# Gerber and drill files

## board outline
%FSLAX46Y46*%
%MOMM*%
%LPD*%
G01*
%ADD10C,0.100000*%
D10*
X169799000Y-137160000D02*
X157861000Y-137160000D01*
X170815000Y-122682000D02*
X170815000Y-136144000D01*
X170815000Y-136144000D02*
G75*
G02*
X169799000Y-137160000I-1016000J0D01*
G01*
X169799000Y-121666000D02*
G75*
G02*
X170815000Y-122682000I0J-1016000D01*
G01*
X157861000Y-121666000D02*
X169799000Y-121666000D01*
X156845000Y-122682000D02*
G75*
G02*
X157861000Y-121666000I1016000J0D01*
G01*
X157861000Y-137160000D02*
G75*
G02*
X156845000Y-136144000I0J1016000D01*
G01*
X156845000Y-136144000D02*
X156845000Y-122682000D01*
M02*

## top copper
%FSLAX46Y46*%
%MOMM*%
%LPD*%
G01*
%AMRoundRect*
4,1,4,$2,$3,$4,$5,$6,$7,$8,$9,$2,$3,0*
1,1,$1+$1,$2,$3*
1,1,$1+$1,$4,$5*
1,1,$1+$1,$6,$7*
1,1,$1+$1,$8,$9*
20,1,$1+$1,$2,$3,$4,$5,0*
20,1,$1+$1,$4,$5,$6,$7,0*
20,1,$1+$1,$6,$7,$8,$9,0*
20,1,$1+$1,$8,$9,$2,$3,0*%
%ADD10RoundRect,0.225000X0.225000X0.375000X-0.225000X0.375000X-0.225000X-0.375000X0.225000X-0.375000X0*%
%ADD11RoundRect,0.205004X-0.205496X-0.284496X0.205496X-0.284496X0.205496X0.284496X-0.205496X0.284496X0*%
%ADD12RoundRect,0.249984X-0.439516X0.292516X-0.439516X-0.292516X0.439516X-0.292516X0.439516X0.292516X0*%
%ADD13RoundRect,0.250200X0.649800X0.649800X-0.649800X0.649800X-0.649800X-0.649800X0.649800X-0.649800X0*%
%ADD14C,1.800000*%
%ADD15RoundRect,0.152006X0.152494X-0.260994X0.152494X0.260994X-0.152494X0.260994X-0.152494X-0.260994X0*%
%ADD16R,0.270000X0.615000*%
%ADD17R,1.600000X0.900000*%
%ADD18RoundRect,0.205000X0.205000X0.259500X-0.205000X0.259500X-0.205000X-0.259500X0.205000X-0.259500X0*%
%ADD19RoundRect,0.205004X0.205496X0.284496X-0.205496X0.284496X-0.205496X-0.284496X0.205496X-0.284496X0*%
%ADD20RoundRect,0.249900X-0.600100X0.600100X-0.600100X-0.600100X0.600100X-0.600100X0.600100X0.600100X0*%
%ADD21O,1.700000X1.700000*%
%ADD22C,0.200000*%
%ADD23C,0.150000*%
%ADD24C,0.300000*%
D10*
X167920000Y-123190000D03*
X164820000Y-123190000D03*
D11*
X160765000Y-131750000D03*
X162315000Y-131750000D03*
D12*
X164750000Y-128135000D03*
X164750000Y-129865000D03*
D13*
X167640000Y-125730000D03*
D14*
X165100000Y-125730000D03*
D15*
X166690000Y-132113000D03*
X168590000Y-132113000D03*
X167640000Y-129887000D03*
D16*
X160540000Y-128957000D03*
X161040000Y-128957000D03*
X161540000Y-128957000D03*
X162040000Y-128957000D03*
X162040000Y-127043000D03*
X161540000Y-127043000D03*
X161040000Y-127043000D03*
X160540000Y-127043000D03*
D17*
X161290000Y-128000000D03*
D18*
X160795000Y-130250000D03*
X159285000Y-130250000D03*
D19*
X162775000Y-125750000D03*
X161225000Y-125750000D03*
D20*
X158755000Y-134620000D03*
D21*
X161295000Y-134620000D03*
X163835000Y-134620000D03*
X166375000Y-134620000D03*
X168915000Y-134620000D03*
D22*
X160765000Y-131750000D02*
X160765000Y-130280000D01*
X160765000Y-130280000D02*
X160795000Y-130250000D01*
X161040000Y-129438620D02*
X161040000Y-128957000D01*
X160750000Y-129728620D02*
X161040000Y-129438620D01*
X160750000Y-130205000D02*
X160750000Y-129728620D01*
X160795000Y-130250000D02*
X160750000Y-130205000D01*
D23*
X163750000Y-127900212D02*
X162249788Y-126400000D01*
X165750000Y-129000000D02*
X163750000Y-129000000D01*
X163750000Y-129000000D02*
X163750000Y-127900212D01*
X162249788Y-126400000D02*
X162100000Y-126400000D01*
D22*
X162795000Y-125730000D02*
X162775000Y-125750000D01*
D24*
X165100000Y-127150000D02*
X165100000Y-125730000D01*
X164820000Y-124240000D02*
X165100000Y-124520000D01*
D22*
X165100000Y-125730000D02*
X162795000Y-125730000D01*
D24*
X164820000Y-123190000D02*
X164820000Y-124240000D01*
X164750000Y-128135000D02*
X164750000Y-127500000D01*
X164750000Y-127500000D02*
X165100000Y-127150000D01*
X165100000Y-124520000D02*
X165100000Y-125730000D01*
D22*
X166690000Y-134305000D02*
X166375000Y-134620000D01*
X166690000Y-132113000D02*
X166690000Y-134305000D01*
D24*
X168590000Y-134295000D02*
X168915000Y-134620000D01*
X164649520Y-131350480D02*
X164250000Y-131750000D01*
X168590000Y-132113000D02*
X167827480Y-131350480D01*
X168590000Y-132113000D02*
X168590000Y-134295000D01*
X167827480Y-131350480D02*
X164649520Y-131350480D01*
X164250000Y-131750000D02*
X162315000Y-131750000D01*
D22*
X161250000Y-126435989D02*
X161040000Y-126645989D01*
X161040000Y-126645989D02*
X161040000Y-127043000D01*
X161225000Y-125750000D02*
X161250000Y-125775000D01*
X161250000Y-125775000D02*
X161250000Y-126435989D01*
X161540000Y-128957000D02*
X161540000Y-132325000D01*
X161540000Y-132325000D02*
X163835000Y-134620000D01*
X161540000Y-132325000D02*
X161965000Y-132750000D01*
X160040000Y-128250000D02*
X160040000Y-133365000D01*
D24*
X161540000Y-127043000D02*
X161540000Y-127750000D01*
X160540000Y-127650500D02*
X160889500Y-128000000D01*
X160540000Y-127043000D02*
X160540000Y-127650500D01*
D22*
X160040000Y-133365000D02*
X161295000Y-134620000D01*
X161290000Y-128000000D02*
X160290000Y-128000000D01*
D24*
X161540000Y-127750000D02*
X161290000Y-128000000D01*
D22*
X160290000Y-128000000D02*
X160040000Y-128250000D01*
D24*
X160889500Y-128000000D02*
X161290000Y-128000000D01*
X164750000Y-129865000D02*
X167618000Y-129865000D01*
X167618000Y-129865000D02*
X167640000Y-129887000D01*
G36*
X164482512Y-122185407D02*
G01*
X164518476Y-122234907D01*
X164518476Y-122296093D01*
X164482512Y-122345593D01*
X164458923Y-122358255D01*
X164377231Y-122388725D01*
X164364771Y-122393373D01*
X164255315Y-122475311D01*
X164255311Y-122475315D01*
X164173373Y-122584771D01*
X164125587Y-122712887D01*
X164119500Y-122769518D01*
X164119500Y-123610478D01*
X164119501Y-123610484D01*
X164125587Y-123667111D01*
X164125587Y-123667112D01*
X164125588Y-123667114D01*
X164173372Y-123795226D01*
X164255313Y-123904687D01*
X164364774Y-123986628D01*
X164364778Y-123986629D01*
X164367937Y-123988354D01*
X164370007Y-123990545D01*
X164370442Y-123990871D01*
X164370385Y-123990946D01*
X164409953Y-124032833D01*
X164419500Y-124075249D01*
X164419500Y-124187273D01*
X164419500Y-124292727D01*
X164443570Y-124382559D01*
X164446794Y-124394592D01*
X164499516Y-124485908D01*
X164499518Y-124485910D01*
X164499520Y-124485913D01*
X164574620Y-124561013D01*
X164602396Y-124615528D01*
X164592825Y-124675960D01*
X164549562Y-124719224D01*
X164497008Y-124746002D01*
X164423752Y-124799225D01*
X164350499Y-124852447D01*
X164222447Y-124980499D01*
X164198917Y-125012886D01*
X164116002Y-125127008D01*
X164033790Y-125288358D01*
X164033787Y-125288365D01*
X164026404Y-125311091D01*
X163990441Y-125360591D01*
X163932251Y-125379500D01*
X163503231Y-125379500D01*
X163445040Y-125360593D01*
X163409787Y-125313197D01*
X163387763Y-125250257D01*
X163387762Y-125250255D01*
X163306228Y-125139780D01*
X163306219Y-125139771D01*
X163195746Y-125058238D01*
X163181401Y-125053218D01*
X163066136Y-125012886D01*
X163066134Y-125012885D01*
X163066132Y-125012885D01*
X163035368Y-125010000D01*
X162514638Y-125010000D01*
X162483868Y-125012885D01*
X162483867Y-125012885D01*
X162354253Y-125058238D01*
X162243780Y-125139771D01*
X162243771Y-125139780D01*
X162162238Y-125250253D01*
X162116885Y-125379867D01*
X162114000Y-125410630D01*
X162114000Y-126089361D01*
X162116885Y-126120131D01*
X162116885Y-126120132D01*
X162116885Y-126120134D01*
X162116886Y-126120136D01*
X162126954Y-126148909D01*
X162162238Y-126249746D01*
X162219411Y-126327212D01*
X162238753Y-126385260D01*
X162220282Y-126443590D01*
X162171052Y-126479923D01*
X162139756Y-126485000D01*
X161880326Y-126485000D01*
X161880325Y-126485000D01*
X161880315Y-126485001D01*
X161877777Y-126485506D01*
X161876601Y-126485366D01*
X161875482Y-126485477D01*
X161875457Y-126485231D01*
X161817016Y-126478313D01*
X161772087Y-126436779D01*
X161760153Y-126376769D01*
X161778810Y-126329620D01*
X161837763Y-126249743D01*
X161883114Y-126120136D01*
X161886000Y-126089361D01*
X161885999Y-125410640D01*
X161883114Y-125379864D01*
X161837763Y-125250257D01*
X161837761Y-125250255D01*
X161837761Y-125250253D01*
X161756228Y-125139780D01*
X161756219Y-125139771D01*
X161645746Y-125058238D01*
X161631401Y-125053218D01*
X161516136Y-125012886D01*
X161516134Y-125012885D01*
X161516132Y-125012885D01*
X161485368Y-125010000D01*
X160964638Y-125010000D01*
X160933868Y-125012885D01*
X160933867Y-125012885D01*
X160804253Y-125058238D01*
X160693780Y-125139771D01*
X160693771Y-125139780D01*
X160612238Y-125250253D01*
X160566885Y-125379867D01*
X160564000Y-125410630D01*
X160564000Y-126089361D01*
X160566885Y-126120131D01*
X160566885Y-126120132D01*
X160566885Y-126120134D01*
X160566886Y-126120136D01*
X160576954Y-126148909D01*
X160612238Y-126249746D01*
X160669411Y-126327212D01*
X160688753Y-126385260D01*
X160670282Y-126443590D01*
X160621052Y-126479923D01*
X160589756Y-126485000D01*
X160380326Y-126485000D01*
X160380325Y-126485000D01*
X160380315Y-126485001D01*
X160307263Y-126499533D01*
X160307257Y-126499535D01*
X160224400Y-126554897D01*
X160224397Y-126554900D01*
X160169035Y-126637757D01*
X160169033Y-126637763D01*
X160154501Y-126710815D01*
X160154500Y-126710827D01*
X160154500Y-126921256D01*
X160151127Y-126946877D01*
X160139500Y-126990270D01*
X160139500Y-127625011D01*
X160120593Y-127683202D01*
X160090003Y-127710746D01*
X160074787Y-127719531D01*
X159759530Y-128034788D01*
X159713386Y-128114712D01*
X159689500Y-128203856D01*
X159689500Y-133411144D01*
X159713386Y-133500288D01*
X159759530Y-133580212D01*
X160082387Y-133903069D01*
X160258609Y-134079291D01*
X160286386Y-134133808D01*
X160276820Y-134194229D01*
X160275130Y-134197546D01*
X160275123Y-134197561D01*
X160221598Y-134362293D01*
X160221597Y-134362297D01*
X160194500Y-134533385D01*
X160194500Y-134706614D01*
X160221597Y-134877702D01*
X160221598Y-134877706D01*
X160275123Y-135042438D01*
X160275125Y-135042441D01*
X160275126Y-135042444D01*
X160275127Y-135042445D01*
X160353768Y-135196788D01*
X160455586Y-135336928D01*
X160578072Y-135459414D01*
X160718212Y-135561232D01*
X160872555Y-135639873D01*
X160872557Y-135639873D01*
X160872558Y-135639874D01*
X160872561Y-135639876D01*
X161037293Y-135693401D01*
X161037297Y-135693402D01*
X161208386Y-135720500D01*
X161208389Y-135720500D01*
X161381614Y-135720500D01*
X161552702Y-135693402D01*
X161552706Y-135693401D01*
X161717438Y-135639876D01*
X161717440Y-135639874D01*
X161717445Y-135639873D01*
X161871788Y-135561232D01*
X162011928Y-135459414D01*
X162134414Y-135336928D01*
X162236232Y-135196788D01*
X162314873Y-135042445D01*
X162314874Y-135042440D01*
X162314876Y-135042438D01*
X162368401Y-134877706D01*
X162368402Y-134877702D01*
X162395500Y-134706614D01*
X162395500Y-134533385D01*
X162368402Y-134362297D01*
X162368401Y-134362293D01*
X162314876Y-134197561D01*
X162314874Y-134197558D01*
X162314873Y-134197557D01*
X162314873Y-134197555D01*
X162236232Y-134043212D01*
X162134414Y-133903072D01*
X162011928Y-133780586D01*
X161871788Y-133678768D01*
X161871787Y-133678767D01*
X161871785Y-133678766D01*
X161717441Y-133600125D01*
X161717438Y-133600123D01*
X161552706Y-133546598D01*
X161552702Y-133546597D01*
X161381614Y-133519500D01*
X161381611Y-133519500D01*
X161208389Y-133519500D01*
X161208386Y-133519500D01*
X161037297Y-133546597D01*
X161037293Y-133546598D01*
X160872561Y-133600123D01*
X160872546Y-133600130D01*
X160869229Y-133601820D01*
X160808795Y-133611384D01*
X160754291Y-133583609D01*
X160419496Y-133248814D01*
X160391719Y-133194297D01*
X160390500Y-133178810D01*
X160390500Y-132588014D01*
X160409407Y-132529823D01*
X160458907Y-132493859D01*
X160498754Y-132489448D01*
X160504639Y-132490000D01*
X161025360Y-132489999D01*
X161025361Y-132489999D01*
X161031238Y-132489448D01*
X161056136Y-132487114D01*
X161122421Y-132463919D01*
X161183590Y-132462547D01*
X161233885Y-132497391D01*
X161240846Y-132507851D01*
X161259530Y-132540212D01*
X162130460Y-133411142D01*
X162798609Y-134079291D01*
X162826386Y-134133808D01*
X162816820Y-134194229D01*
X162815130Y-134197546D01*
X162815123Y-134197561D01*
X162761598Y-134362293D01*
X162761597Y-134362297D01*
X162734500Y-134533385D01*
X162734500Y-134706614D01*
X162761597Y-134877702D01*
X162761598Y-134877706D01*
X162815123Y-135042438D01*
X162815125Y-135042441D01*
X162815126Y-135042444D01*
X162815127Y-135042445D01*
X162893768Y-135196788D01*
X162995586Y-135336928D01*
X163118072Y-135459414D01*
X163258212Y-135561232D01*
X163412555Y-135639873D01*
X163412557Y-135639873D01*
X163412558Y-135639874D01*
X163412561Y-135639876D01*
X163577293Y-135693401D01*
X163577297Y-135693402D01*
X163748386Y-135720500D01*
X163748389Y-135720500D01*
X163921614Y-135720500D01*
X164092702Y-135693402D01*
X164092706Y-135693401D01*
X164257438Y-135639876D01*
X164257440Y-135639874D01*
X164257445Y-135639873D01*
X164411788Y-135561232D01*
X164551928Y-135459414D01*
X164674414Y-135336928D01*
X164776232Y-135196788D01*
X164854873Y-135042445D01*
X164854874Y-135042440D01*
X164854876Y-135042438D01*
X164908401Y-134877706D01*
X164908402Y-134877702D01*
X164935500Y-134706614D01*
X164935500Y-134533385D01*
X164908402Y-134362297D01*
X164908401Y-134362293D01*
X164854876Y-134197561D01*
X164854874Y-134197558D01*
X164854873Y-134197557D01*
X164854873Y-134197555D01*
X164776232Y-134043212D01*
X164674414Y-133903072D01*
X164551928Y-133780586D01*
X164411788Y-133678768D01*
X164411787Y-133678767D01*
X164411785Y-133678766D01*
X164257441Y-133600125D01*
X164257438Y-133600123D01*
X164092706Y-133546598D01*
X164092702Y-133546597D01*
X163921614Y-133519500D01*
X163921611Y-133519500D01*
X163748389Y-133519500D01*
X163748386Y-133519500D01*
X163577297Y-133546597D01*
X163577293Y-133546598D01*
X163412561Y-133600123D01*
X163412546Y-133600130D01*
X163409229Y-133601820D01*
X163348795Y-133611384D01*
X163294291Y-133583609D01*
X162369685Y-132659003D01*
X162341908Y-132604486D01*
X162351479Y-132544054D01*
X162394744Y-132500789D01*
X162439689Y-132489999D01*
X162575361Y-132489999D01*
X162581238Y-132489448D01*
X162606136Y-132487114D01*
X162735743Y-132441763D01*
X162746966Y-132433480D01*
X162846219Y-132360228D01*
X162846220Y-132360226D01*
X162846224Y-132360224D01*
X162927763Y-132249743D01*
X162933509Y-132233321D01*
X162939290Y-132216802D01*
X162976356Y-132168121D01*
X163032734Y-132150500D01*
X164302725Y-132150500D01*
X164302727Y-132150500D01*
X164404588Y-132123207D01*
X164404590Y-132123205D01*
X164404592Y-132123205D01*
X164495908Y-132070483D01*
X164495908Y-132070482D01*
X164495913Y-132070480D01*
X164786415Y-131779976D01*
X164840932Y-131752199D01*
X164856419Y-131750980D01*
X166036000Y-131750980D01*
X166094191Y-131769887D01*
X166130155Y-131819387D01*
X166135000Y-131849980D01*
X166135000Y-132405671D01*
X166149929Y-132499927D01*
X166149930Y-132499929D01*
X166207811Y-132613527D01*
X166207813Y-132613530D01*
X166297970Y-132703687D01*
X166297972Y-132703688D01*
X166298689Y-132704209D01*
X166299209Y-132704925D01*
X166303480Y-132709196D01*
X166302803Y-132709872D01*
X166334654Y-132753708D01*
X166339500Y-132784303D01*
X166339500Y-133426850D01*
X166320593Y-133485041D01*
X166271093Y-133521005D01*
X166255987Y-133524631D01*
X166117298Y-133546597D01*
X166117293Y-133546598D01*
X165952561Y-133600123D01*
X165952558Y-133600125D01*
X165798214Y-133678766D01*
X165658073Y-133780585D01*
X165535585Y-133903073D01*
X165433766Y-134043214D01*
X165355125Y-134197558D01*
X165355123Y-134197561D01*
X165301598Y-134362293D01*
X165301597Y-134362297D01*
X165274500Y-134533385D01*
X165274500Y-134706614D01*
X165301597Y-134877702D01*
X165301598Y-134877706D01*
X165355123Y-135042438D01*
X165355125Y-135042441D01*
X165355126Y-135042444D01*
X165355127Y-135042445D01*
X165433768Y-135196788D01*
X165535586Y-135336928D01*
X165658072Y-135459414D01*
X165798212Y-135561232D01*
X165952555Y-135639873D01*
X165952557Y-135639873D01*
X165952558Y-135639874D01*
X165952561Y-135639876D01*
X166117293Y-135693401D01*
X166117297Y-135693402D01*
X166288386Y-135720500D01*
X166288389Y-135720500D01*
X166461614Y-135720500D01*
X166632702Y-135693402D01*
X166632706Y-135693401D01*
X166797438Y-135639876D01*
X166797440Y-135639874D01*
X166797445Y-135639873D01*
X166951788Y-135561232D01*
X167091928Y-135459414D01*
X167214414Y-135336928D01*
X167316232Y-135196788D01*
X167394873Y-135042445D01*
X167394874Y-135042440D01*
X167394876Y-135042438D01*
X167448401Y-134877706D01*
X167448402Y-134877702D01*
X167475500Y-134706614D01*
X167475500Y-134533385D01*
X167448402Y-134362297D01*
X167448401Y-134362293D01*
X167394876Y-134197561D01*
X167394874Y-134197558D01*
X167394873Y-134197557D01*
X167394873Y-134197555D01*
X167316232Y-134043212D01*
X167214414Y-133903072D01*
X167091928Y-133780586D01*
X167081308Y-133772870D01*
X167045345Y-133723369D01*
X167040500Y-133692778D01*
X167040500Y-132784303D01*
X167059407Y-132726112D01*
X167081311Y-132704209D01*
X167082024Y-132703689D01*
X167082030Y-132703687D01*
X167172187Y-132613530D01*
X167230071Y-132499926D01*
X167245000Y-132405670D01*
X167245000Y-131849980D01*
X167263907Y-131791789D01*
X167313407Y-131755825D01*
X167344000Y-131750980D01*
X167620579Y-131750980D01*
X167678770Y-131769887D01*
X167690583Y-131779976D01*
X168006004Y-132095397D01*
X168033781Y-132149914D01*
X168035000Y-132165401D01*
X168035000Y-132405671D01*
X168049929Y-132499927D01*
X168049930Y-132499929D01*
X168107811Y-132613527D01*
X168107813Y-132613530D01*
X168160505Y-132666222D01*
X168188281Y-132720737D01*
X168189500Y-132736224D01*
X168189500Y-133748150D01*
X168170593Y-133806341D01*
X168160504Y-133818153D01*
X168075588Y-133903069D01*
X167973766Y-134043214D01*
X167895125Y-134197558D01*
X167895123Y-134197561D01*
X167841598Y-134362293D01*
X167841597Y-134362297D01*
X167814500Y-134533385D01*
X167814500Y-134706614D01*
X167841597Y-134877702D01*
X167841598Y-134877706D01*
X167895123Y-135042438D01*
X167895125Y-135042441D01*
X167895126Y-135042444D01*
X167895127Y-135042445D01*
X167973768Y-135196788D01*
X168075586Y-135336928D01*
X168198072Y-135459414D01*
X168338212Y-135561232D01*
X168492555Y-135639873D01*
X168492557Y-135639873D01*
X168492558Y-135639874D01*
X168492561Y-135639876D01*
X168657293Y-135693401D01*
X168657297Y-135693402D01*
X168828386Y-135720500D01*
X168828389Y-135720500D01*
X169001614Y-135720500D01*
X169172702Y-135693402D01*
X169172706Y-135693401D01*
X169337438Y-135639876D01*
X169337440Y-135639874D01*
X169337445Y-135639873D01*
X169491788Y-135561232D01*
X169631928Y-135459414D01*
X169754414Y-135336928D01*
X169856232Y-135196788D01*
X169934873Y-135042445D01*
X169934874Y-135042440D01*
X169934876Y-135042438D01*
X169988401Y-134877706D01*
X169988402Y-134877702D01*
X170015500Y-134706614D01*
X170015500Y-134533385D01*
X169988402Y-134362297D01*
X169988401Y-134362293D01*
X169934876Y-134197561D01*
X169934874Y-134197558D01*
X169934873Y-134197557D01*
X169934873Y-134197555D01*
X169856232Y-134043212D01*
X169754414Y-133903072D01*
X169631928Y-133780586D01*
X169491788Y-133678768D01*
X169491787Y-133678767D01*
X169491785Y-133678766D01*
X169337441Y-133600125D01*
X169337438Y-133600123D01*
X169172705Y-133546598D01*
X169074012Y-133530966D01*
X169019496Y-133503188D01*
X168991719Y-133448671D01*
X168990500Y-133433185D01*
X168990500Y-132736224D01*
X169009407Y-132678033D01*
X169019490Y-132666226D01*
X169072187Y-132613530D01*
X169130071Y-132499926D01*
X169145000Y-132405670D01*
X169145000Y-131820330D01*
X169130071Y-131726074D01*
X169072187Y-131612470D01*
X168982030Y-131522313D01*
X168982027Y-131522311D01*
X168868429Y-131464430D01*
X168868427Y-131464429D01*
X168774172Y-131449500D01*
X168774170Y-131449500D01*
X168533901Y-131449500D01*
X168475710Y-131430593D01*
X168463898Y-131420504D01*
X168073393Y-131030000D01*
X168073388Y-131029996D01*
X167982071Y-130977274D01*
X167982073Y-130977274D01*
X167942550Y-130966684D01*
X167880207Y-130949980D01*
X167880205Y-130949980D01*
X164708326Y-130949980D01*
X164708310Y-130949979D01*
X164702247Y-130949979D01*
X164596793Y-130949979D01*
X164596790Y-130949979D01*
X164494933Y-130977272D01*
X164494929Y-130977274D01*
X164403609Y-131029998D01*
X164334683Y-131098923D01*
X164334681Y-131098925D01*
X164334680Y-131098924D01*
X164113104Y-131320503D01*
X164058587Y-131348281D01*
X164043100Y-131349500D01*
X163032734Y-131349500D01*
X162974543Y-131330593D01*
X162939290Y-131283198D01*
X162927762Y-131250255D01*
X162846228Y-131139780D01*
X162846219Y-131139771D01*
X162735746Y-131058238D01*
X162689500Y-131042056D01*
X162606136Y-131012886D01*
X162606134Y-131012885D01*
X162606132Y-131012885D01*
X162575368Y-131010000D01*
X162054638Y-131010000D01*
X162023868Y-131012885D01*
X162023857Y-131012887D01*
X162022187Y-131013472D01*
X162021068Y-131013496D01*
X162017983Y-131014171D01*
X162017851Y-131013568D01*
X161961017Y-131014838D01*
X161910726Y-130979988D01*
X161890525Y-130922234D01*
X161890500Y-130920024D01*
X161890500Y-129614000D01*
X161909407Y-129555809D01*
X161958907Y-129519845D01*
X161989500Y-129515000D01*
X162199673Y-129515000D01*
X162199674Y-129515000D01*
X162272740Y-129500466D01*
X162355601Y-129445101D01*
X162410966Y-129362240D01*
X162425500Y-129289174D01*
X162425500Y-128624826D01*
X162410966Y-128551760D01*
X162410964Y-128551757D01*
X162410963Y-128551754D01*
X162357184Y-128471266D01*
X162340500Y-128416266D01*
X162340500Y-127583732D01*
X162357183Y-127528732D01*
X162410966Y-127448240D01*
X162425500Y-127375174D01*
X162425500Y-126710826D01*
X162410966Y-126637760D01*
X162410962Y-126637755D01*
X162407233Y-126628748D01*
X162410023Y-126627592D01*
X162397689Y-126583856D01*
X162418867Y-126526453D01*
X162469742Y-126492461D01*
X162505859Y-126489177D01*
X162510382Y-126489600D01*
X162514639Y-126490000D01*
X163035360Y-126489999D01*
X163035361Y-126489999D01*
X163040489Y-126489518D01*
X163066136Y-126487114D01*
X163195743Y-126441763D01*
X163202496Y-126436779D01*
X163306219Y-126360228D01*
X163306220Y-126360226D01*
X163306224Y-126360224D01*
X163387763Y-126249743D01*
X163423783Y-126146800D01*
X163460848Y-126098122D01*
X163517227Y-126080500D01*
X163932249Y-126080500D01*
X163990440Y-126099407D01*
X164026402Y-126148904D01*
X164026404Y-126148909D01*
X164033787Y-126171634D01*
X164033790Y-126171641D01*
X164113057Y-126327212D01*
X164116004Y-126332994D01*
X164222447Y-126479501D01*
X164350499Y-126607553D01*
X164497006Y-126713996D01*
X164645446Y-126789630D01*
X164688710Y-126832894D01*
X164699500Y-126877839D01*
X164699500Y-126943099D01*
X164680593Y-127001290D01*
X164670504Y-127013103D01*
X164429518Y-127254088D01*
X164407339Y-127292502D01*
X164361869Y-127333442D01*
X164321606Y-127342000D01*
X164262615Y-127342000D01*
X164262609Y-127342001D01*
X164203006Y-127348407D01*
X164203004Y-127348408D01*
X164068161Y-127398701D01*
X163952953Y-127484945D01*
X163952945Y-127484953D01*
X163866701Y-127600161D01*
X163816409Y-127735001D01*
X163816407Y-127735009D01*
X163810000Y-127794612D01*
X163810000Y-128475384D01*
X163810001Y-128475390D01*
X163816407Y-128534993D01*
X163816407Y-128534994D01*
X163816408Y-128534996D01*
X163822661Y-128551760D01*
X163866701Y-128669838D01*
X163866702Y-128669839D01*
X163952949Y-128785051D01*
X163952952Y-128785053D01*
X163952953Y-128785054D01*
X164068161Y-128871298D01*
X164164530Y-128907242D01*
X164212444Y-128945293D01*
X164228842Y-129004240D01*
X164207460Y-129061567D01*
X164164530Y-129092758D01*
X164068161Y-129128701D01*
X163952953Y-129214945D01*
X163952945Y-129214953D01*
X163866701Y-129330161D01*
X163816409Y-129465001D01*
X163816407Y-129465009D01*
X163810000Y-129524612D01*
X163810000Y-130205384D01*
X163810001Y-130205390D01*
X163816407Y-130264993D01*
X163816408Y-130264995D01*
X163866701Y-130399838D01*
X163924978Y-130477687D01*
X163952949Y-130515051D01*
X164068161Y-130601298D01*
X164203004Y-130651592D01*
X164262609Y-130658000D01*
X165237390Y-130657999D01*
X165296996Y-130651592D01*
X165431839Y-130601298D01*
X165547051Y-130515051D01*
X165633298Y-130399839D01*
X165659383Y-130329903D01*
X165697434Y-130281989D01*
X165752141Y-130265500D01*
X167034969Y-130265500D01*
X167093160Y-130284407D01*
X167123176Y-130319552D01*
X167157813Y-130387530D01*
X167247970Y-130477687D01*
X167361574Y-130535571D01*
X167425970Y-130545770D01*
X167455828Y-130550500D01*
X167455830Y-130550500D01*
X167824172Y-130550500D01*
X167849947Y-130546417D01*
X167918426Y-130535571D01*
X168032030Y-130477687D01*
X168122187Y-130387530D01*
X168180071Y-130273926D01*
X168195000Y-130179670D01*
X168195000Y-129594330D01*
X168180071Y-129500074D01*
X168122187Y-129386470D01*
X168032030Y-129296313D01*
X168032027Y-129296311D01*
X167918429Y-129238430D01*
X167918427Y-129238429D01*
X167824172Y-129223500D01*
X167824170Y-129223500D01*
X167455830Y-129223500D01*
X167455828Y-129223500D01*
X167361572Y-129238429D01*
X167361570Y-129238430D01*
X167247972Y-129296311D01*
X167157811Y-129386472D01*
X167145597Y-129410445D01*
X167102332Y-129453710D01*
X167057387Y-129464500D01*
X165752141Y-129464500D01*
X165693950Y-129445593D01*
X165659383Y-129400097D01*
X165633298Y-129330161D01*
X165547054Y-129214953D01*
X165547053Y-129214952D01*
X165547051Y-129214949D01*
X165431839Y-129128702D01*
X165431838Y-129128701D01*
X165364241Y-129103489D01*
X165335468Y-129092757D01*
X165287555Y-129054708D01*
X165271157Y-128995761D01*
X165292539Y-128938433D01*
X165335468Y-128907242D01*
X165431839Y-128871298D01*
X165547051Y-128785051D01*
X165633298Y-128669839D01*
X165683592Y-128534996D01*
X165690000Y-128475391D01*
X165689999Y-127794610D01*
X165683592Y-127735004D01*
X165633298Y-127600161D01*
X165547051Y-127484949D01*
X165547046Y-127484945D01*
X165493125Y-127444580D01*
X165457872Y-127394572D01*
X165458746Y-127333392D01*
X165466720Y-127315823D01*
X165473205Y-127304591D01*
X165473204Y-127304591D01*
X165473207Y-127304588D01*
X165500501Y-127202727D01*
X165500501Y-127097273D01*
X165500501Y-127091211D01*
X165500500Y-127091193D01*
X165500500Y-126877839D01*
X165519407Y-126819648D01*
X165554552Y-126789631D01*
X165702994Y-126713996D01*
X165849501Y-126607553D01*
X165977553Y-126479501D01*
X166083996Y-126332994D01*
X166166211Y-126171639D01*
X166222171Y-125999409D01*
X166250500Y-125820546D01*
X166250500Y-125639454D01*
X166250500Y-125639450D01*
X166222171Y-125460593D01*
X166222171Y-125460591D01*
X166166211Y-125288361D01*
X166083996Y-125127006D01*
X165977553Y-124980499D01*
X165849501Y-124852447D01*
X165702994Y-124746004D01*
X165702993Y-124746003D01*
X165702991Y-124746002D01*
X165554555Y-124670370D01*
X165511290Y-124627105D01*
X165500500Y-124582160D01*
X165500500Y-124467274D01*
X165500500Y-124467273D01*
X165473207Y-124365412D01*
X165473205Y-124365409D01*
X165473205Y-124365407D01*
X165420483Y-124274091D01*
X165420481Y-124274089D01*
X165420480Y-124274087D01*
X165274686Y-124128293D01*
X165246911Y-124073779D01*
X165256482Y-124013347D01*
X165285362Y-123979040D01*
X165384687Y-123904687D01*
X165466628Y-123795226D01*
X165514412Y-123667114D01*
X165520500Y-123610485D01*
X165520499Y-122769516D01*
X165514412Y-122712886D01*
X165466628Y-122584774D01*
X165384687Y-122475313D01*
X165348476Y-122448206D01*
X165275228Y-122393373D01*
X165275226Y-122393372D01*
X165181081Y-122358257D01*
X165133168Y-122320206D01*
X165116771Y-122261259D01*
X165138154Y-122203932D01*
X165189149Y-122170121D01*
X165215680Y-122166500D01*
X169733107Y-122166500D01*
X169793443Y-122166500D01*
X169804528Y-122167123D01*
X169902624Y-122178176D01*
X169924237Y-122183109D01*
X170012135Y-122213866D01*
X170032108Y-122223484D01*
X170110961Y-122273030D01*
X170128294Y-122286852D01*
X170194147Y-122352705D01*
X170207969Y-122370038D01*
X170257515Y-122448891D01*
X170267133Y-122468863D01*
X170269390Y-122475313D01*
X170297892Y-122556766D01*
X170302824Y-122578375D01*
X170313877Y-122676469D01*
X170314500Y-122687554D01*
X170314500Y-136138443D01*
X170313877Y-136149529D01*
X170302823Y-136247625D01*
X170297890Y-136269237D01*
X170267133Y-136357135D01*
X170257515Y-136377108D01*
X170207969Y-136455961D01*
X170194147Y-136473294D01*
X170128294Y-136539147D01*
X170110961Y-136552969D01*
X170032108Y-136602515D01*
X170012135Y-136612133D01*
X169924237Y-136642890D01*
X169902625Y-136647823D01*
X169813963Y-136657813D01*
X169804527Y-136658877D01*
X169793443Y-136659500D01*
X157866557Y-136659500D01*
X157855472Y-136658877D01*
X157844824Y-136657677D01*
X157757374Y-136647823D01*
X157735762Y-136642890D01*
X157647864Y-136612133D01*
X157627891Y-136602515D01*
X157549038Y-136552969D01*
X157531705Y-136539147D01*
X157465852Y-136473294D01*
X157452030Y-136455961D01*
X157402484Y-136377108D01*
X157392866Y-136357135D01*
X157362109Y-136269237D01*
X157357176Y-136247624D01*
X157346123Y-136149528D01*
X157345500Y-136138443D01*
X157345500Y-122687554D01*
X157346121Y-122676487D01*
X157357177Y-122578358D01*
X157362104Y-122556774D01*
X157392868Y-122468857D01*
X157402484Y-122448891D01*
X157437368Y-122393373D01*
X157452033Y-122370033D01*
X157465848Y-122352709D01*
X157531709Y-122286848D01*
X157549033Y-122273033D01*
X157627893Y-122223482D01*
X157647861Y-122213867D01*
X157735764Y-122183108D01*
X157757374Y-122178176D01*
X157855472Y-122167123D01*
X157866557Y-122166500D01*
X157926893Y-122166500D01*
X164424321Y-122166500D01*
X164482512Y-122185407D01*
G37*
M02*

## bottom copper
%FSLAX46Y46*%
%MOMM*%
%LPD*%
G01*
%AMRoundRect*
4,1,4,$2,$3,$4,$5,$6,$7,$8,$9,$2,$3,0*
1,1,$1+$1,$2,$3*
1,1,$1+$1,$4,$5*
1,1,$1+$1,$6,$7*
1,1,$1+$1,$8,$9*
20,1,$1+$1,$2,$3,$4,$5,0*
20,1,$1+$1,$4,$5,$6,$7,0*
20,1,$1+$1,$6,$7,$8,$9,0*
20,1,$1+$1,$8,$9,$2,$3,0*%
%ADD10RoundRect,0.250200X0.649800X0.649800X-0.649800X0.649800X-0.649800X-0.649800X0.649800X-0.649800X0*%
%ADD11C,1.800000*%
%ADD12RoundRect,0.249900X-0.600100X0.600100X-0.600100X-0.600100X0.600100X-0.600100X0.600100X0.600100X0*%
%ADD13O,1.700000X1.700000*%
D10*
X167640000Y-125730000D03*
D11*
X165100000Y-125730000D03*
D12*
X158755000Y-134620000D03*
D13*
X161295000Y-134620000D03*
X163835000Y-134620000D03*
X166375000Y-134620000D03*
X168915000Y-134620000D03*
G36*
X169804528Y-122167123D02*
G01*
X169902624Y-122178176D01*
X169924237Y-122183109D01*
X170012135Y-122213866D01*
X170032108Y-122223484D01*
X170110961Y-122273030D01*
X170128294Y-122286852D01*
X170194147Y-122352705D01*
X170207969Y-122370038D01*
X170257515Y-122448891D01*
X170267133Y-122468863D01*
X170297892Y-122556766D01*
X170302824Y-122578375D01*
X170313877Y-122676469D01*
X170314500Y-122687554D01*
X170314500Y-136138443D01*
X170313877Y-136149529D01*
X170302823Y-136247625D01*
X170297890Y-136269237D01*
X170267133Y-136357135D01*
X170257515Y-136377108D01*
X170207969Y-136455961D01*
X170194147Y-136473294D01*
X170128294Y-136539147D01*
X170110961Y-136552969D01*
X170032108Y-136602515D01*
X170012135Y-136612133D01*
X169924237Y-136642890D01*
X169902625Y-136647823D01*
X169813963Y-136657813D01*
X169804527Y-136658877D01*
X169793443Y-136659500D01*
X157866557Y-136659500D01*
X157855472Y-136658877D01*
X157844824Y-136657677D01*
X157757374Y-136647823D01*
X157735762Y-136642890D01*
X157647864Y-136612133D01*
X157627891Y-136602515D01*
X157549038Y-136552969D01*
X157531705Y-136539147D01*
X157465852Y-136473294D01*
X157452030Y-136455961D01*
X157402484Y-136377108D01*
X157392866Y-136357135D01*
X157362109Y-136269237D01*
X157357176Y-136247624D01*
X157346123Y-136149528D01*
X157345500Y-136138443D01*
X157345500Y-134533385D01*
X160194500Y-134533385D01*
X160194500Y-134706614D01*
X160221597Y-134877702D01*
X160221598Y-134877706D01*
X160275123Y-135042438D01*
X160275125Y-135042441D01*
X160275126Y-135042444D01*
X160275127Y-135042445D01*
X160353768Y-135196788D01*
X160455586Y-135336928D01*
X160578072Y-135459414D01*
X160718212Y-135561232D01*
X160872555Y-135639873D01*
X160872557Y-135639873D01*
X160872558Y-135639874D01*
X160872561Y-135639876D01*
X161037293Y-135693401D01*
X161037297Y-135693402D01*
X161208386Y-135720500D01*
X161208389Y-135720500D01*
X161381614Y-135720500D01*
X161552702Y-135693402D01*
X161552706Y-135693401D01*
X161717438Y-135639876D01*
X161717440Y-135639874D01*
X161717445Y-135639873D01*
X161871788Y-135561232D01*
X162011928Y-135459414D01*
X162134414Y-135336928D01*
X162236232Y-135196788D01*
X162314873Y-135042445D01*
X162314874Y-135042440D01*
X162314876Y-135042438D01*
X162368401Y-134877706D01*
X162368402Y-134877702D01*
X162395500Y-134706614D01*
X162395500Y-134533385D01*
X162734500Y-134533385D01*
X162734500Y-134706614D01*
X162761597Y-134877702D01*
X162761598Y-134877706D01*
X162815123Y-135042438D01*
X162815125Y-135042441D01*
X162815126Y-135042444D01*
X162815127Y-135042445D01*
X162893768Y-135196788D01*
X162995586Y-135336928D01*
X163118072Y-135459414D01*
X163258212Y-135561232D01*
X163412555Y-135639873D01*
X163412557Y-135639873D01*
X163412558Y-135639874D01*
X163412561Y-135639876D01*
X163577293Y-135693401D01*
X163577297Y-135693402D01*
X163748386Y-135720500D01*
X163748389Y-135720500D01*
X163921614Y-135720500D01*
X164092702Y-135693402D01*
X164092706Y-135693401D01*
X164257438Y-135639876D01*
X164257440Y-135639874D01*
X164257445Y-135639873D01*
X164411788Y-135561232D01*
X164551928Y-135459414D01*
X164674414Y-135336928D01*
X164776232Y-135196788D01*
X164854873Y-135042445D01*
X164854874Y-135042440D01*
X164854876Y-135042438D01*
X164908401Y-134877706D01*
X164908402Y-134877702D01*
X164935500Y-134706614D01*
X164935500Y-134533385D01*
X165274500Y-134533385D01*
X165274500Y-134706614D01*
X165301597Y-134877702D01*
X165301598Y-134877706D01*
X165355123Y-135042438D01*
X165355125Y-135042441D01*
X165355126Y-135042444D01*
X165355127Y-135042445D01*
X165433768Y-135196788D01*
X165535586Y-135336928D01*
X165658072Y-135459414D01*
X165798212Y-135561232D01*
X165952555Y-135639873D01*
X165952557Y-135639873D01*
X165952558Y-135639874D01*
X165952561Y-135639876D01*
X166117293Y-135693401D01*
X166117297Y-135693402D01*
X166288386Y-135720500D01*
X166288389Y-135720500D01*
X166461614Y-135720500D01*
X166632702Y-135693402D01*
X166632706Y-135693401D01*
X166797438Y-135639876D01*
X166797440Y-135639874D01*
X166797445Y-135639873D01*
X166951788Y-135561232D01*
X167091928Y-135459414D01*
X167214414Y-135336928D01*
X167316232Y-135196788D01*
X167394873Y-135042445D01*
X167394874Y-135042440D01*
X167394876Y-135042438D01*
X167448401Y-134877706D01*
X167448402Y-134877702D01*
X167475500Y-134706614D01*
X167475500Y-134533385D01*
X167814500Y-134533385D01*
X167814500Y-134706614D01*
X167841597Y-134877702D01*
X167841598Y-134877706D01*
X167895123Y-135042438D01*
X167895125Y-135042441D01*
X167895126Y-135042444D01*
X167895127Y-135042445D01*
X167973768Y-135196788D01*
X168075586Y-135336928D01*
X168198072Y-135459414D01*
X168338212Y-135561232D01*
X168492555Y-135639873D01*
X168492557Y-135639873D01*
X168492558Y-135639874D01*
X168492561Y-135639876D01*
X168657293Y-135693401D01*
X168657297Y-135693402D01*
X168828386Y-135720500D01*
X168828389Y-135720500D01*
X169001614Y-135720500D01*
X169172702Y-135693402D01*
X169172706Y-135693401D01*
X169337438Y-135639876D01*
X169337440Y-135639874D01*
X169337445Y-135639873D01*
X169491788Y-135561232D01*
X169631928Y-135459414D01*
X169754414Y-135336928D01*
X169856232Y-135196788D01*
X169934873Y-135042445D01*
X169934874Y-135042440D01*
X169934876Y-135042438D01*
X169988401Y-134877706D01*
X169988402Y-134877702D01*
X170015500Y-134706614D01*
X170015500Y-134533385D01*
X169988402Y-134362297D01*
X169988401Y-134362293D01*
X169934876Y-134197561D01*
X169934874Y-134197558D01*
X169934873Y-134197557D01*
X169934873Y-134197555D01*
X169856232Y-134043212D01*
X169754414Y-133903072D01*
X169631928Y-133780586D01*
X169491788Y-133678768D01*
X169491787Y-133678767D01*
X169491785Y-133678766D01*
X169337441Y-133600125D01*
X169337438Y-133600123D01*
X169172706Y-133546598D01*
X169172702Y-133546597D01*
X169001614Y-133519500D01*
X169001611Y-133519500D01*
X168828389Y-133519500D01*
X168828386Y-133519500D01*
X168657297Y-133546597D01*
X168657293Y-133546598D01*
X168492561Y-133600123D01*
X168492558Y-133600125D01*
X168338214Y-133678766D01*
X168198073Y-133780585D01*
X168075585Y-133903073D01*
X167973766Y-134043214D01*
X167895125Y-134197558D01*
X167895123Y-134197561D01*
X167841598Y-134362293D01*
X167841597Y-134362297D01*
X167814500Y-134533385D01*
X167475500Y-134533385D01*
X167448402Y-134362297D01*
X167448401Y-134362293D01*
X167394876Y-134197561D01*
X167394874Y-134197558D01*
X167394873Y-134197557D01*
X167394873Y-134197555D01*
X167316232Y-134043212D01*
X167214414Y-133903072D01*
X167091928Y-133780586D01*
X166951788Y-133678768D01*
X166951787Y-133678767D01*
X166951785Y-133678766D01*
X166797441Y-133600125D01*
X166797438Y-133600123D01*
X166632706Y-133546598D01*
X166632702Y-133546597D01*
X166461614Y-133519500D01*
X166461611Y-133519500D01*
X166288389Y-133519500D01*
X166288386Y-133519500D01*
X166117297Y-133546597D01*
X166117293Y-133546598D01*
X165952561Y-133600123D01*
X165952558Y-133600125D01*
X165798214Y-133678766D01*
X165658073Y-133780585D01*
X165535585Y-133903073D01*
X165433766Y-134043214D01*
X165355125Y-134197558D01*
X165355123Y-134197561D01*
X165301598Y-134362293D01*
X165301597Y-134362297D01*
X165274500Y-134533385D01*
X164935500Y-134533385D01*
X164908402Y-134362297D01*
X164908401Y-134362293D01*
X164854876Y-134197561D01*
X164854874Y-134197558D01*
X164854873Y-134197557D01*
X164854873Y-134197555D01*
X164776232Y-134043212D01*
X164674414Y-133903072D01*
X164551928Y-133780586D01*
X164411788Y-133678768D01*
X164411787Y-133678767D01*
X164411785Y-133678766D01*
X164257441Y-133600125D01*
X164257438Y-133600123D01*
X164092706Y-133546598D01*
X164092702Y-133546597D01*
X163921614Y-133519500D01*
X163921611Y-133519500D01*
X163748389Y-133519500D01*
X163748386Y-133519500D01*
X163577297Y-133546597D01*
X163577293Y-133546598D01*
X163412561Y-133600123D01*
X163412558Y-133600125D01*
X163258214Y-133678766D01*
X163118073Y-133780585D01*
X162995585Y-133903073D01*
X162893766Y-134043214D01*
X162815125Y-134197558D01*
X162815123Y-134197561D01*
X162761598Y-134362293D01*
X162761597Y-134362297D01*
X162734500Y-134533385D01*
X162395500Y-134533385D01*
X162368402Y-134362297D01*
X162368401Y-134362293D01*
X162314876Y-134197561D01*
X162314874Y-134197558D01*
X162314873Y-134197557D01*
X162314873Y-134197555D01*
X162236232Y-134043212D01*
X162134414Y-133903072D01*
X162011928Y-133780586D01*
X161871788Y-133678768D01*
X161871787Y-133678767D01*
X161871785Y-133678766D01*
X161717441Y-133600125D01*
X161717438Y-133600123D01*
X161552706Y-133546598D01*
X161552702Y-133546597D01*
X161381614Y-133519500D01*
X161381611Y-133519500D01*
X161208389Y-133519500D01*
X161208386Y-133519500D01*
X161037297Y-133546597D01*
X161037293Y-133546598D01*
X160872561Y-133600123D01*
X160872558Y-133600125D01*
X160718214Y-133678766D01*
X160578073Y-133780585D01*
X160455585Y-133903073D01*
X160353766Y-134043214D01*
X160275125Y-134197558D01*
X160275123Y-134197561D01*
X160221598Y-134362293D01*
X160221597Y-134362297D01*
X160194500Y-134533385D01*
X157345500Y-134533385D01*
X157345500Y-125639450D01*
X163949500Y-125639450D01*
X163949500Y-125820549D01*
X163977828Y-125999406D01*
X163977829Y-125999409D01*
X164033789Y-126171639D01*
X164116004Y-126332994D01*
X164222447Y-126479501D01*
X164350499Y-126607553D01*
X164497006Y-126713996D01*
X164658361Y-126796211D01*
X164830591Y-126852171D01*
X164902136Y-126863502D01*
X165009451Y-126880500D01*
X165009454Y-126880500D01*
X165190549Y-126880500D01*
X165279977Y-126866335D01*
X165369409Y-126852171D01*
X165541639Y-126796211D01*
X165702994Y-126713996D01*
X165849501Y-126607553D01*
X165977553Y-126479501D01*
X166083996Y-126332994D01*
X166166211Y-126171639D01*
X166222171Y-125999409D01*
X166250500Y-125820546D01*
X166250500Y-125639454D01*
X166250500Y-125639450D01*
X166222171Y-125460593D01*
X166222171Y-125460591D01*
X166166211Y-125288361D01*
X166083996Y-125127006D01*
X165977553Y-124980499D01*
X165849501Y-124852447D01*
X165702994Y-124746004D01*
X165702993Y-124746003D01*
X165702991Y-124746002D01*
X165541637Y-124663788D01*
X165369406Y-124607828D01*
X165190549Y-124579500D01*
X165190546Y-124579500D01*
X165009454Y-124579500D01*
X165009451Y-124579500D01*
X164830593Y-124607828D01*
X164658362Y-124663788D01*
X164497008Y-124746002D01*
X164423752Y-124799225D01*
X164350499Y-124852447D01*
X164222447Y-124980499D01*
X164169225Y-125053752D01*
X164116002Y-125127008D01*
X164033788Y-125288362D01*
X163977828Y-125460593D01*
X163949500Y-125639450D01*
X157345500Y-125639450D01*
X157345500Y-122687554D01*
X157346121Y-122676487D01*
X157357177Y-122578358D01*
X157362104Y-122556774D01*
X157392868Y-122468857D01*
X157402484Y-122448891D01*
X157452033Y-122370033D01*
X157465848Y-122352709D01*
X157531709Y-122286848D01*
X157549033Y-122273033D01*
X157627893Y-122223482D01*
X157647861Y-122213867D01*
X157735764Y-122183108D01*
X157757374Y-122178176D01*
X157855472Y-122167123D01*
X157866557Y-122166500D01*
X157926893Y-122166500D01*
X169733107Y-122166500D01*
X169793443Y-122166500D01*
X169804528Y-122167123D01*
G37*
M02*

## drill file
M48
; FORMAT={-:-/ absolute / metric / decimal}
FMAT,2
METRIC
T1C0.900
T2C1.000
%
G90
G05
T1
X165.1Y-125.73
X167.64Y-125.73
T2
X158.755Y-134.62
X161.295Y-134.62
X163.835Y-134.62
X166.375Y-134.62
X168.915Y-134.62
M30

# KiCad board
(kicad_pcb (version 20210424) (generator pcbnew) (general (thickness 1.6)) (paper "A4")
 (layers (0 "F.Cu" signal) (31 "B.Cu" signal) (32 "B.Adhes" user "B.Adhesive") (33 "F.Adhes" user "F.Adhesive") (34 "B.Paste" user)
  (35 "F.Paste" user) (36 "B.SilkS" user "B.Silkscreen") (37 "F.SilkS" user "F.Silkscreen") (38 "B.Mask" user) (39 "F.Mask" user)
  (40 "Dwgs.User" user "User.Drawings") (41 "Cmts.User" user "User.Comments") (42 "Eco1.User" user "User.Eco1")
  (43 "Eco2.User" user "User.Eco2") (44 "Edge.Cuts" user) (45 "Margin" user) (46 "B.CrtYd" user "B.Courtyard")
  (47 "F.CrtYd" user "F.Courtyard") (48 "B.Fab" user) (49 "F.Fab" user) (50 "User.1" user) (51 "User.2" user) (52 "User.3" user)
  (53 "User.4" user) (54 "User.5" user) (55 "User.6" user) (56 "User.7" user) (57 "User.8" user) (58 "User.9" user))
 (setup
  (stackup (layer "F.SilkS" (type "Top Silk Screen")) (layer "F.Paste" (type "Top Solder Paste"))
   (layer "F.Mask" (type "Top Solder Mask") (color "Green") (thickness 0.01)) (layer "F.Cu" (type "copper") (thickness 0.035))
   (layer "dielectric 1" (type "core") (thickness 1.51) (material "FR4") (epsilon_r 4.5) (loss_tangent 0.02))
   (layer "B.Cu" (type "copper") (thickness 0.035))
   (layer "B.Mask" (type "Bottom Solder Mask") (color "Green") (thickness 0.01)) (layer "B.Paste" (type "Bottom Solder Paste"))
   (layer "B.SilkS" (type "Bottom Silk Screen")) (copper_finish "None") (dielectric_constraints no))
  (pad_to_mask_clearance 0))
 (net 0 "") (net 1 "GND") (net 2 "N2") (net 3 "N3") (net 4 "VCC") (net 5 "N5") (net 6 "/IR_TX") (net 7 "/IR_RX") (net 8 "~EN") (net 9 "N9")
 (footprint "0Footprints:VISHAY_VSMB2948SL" (layer "F.Cu") (at 166.37 123.19 180)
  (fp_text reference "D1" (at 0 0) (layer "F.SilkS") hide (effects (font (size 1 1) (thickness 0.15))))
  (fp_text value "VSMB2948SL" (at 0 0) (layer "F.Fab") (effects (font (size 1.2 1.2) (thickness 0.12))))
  (pad "1" smd roundrect (at -1.55 0 180) (size 0.9 1.2) (layers "F.Cu" "F.Paste" "F.Mask") (roundrect_rratio 0.25) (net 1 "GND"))
  (pad "2" smd roundrect (at 1.55 0 180) (size 0.9 1.2) (layers "F.Cu" "F.Paste" "F.Mask") (roundrect_rratio 0.25) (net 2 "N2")))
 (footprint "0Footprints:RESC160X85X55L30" (layer "F.Cu") (at 161.54 131.75)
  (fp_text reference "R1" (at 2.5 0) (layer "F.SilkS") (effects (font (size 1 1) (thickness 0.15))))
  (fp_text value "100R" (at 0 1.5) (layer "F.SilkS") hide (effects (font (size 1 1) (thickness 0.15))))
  (pad "1" smd roundrect (at -0.775 0) (size 0.821 0.979) (layers "F.Cu" "F.Paste" "F.Mask") (roundrect_rratio 0.2497003654) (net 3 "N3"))
  (pad "2" smd roundrect (at 0.775 0) (size 0.821 0.979) (layers "F.Cu" "F.Paste" "F.Mask") (roundrect_rratio 0.2497003654) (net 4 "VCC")))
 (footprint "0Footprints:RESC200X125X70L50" (layer "F.Cu") (at 164.75 129 -90)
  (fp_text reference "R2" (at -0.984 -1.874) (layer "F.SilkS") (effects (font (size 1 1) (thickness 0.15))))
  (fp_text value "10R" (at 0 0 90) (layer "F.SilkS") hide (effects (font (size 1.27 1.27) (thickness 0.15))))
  (pad "1" smd roundrect (at -0.865 0 270) (size 1.085 1.379) (layers "F.Cu" "F.Paste" "F.Mask") (roundrect_rratio 0.2304) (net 2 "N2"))
  (pad "2" smd roundrect (at 0.865 0 270) (size 1.085 1.379) (layers "F.Cu" "F.Paste" "F.Mask") (roundrect_rratio 0.2304) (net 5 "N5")))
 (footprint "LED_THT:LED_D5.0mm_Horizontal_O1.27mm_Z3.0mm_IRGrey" (layer "F.Cu") (at 167.64 125.73 180)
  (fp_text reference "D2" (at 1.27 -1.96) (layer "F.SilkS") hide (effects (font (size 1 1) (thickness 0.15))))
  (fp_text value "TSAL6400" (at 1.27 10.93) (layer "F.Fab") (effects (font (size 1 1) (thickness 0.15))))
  (pad "1" thru_hole roundrect locked (at 0 0 180) (size 1.8 1.8) (drill 0.9) (layers *.Cu *.Mask) (roundrect_rratio 0.139) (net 1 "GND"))
  (pad "2" thru_hole circle locked (at 2.54 0 180) (size 1.8 1.8) (drill 0.9) (layers *.Cu *.Mask) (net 2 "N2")))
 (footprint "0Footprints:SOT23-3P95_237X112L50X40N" (layer "F.Cu") (at 167.64 131)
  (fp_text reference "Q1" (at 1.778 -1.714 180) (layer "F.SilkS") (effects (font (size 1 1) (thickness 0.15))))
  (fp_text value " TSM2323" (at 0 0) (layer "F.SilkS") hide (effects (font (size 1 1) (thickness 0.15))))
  (pad "1" smd roundrect (at -0.95 1.113 90) (size 0.826 0.609) (layers "F.Cu" "F.Paste" "F.Mask") (roundrect_rratio 0.2495993432)
   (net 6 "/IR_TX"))
  (pad "2" smd roundrect (at 0.95 1.113 90) (size 0.826 0.609) (layers "F.Cu" "F.Paste" "F.Mask") (roundrect_rratio 0.2495993432)
   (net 4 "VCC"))
  (pad "3" smd roundrect (at 0 -1.113 90) (size 0.826 0.609) (layers "F.Cu" "F.Paste" "F.Mask") (roundrect_rratio 0.2495993432) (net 5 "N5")))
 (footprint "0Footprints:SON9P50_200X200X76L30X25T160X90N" (layer "F.Cu") (at 161.29 128)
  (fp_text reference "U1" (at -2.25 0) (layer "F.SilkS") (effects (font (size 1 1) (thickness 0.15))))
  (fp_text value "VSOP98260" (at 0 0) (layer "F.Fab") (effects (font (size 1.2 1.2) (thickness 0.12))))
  (pad "" smd roundrect (at -0.348 -0.049 90) (size 0.538 0.565) (layers "F.Paste") (roundrect_rratio 0.25))
  (pad "" smd roundrect (at 0.4 0 90) (size 0.636 0.668) (layers "F.Paste") (roundrect_rratio 0.25))
  (pad "1" smd rect (at -0.75 0.957 90) (size 0.615 0.27) (layers "F.Cu" "F.Paste" "F.Mask"))
  (pad "2" smd rect (at -0.25 0.957 90) (size 0.615 0.27) (layers "F.Cu" "F.Paste" "F.Mask") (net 3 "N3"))
  (pad "3" smd rect (at 0.25 0.957 90) (size 0.615 0.27) (layers "F.Cu" "F.Paste" "F.Mask") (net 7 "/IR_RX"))
  (pad "4" smd rect (at 0.75 0.957 90) (size 0.615 0.27) (layers "F.Cu" "F.Paste" "F.Mask"))
  (pad "5" smd rect (at 0.75 -0.957 90) (size 0.615 0.27) (layers "F.Cu" "F.Paste" "F.Mask"))
  (pad "6" smd rect (at 0.25 -0.957 90) (size 0.615 0.27) (layers "F.Cu" "F.Paste" "F.Mask") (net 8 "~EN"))
  (pad "7" smd rect (at -0.25 -0.957 90) (size 0.615 0.27) (layers "F.Cu" "F.Paste" "F.Mask") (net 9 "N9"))
  (pad "8" smd rect (at -0.75 -0.957 90) (size 0.615 0.27) (layers "F.Cu" "F.Paste" "F.Mask") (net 8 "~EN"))
  (pad "9" smd rect (at 0 0 90) (size 0.9 1.6) (layers "F.Cu" "F.Mask") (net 8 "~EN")))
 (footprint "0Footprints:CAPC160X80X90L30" (layer "F.Cu") (at 160.04 130.25 180)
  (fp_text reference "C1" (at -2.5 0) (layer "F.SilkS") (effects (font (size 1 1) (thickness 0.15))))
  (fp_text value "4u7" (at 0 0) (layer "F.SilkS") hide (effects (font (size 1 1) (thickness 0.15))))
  (pad "1" smd roundrect (at -0.755 0 180) (size 0.82 0.929) (layers "F.Cu" "F.Paste" "F.Mask") (roundrect_rratio 0.25) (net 3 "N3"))
  (pad "2" smd roundrect (at 0.755 0 180) (size 0.82 0.929) (layers "F.Cu" "F.Paste" "F.Mask") (roundrect_rratio 0.25) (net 1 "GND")))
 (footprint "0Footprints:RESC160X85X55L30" (layer "F.Cu") (at 162 125.75 180)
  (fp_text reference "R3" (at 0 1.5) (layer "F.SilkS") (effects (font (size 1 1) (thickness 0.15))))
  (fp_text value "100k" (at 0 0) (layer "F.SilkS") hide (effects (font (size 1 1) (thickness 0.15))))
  (pad "1" smd roundrect (at -0.775 0 180) (size 0.821 0.979) (layers "F.Cu" "F.Paste" "F.Mask") (roundrect_rratio 0.2497003654)
   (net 2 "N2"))
  (pad "2" smd roundrect (at 0.775 0 180) (size 0.821 0.979) (layers "F.Cu" "F.Paste" "F.Mask") (roundrect_rratio 0.2497003654) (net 9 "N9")))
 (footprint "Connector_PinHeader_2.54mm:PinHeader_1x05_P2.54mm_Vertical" (layer "B.Cu") (at 158.755 134.62 -90)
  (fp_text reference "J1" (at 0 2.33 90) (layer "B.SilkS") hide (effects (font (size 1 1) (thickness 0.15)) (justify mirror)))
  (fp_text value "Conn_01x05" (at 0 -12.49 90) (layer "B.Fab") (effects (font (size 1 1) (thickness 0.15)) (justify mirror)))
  (pad "1" thru_hole roundrect locked (at 0 0 270) (size 1.7 1.7) (drill 1) (layers *.Cu *.Mask) (roundrect_rratio 0.147) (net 1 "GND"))
  (pad "2" thru_hole oval locked (at 0 -2.54 270) (size 1.7 1.7) (drill 1) (layers *.Cu *.Mask) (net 8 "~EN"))
  (pad "3" thru_hole oval locked (at 0 -5.08 270) (size 1.7 1.7) (drill 1) (layers *.Cu *.Mask) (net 7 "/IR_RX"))
  (pad "4" thru_hole oval locked (at 0 -7.62 270) (size 1.7 1.7) (drill 1) (layers *.Cu *.Mask) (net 6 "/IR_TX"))
  (pad "5" thru_hole oval locked (at 0 -10.16 270) (size 1.7 1.7) (drill 1) (layers *.Cu *.Mask) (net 4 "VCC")))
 (gr_line (start 169.799 137.16) (end 157.861 137.16) (layer "Edge.Cuts") (width 0.1))
 (gr_line (start 170.815 122.682) (end 170.815 136.144) (layer "Edge.Cuts") (width 0.1))
 (gr_arc (start 169.799 136.144) (end 170.815 136.144) (angle 90) (layer "Edge.Cuts") (width 0.1))
 (gr_arc (start 169.799 122.682) (end 169.799 121.666) (angle 90) (layer "Edge.Cuts") (width 0.1))
 (gr_line (start 157.861 121.666) (end 169.799 121.666) (layer "Edge.Cuts") (width 0.1))
 (gr_arc (start 157.861 122.682) (end 156.845 122.682) (angle 90) (layer "Edge.Cuts") (width 0.1))
 (gr_arc (start 157.861 136.144) (end 157.861 137.16) (angle 90) (layer "Edge.Cuts") (width 0.1))
 (gr_line (start 156.845 136.144) (end 156.845 122.682) (layer "Edge.Cuts") (width 0.1))
 (segment (start 160.765 131.75) (end 160.765 130.28) (width 0.2) (layer "F.Cu") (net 3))
 (segment (start 160.765 130.28) (end 160.795 130.25) (width 0.2) (layer "F.Cu") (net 3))
 (segment (start 161.04 129.43862) (end 161.04 128.957) (width 0.2) (layer "F.Cu") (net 3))
 (segment (start 160.75 129.72862) (end 161.04 129.43862) (width 0.2) (layer "F.Cu") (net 3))
 (segment (start 160.75 130.205) (end 160.75 129.72862) (width 0.2) (layer "F.Cu") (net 3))
 (segment (start 160.795 130.25) (end 160.75 130.205) (width 0.2) (layer "F.Cu") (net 3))
 (segment (start 163.75 127.900212) (end 162.249788 126.4) (width 0.15) (layer "F.Cu") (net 1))
 (segment (start 165.75 129) (end 163.75 129) (width 0.15) (layer "F.Cu") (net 1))
 (segment (start 163.75 129) (end 163.75 127.900212) (width 0.15) (layer "F.Cu") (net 1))
 (segment (start 162.249788 126.4) (end 162.1 126.4) (width 0.15) (layer "F.Cu") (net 1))
 (segment (start 162.795 125.73) (end 162.775 125.75) (width 0.2) (layer "F.Cu") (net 2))
 (segment (start 165.1 127.15) (end 165.1 125.73) (width 0.3) (layer "F.Cu") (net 2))
 (segment (start 164.82 124.24) (end 165.1 124.52) (width 0.3) (layer "F.Cu") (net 2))
 (segment (start 165.1 125.73) (end 162.795 125.73) (width 0.2) (layer "F.Cu") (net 2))
 (segment (start 164.82 123.19) (end 164.82 124.24) (width 0.3) (layer "F.Cu") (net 2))
 (segment (start 164.75 128.135) (end 164.75 127.5) (width 0.3) (layer "F.Cu") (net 2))
 (segment (start 164.75 127.5) (end 165.1 127.15) (width 0.3) (layer "F.Cu") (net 2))
 (segment (start 165.1 124.52) (end 165.1 125.73) (width 0.3) (layer "F.Cu") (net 2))
 (segment (start 166.69 134.305) (end 166.375 134.62) (width 0.2) (layer "F.Cu") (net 6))
 (segment (start 166.69 132.113) (end 166.69 134.305) (width 0.2) (layer "F.Cu") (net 6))
 (segment (start 168.59 134.295) (end 168.915 134.62) (width 0.3) (layer "F.Cu") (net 4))
 (segment (start 164.64952 131.35048) (end 164.25 131.75) (width 0.3) (layer "F.Cu") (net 4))
 (segment (start 168.59 132.113) (end 167.82748 131.35048) (width 0.3) (layer "F.Cu") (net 4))
 (segment (start 168.59 132.113) (end 168.59 134.295) (width 0.3) (layer "F.Cu") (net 4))
 (segment (start 167.82748 131.35048) (end 164.64952 131.35048) (width 0.3) (layer "F.Cu") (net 4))
 (segment (start 164.25 131.75) (end 162.315 131.75) (width 0.3) (layer "F.Cu") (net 4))
 (segment (start 161.25 126.435989) (end 161.04 126.645989) (width 0.2) (layer "F.Cu") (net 9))
 (segment (start 161.04 126.645989) (end 161.04 127.043) (width 0.2) (layer "F.Cu") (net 9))
 (segment (start 161.225 125.75) (end 161.25 125.775) (width 0.2) (layer "F.Cu") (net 9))
 (segment (start 161.25 125.775) (end 161.25 126.435989) (width 0.2) (layer "F.Cu") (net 9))
 (segment (start 161.54 128.957) (end 161.54 132.325) (width 0.2) (layer "F.Cu") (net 7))
 (segment (start 161.54 132.325) (end 163.835 134.62) (width 0.2) (layer "F.Cu") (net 7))
 (segment (start 161.54 132.325) (end 161.965 132.75) (width 0.2) (layer "F.Cu") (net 7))
 (segment (start 160.04 128.25) (end 160.04 133.365) (width 0.2) (layer "F.Cu") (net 8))
 (segment (start 161.54 127.043) (end 161.54 127.75) (width 0.3) (layer "F.Cu") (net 8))
 (segment (start 160.54 127.6505) (end 160.8895 128) (width 0.3) (layer "F.Cu") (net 8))
 (segment (start 160.54 127.043) (end 160.54 127.6505) (width 0.3) (layer "F.Cu") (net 8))
 (segment (start 160.04 133.365) (end 161.295 134.62) (width 0.2) (layer "F.Cu") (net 8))
 (segment (start 161.29 128) (end 160.29 128) (width 0.2) (layer "F.Cu") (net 8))
 (segment (start 161.54 127.75) (end 161.29 128) (width 0.3) (layer "F.Cu") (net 8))
 (segment (start 160.29 128) (end 160.04 128.25) (width 0.2) (layer "F.Cu") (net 8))
 (segment (start 160.8895 128) (end 161.29 128) (width 0.3) (layer "F.Cu") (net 8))
 (segment (start 164.75 129.865) (end 167.618 129.865) (width 0.3) (layer "F.Cu") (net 5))
 (segment (start 167.618 129.865) (end 167.64 129.887) (width 0.3) (layer "F.Cu") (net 5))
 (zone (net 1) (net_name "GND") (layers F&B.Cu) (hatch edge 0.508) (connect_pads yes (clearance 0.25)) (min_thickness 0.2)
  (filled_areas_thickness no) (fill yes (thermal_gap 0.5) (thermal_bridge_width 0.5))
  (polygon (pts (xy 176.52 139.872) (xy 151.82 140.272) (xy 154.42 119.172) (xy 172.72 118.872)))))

